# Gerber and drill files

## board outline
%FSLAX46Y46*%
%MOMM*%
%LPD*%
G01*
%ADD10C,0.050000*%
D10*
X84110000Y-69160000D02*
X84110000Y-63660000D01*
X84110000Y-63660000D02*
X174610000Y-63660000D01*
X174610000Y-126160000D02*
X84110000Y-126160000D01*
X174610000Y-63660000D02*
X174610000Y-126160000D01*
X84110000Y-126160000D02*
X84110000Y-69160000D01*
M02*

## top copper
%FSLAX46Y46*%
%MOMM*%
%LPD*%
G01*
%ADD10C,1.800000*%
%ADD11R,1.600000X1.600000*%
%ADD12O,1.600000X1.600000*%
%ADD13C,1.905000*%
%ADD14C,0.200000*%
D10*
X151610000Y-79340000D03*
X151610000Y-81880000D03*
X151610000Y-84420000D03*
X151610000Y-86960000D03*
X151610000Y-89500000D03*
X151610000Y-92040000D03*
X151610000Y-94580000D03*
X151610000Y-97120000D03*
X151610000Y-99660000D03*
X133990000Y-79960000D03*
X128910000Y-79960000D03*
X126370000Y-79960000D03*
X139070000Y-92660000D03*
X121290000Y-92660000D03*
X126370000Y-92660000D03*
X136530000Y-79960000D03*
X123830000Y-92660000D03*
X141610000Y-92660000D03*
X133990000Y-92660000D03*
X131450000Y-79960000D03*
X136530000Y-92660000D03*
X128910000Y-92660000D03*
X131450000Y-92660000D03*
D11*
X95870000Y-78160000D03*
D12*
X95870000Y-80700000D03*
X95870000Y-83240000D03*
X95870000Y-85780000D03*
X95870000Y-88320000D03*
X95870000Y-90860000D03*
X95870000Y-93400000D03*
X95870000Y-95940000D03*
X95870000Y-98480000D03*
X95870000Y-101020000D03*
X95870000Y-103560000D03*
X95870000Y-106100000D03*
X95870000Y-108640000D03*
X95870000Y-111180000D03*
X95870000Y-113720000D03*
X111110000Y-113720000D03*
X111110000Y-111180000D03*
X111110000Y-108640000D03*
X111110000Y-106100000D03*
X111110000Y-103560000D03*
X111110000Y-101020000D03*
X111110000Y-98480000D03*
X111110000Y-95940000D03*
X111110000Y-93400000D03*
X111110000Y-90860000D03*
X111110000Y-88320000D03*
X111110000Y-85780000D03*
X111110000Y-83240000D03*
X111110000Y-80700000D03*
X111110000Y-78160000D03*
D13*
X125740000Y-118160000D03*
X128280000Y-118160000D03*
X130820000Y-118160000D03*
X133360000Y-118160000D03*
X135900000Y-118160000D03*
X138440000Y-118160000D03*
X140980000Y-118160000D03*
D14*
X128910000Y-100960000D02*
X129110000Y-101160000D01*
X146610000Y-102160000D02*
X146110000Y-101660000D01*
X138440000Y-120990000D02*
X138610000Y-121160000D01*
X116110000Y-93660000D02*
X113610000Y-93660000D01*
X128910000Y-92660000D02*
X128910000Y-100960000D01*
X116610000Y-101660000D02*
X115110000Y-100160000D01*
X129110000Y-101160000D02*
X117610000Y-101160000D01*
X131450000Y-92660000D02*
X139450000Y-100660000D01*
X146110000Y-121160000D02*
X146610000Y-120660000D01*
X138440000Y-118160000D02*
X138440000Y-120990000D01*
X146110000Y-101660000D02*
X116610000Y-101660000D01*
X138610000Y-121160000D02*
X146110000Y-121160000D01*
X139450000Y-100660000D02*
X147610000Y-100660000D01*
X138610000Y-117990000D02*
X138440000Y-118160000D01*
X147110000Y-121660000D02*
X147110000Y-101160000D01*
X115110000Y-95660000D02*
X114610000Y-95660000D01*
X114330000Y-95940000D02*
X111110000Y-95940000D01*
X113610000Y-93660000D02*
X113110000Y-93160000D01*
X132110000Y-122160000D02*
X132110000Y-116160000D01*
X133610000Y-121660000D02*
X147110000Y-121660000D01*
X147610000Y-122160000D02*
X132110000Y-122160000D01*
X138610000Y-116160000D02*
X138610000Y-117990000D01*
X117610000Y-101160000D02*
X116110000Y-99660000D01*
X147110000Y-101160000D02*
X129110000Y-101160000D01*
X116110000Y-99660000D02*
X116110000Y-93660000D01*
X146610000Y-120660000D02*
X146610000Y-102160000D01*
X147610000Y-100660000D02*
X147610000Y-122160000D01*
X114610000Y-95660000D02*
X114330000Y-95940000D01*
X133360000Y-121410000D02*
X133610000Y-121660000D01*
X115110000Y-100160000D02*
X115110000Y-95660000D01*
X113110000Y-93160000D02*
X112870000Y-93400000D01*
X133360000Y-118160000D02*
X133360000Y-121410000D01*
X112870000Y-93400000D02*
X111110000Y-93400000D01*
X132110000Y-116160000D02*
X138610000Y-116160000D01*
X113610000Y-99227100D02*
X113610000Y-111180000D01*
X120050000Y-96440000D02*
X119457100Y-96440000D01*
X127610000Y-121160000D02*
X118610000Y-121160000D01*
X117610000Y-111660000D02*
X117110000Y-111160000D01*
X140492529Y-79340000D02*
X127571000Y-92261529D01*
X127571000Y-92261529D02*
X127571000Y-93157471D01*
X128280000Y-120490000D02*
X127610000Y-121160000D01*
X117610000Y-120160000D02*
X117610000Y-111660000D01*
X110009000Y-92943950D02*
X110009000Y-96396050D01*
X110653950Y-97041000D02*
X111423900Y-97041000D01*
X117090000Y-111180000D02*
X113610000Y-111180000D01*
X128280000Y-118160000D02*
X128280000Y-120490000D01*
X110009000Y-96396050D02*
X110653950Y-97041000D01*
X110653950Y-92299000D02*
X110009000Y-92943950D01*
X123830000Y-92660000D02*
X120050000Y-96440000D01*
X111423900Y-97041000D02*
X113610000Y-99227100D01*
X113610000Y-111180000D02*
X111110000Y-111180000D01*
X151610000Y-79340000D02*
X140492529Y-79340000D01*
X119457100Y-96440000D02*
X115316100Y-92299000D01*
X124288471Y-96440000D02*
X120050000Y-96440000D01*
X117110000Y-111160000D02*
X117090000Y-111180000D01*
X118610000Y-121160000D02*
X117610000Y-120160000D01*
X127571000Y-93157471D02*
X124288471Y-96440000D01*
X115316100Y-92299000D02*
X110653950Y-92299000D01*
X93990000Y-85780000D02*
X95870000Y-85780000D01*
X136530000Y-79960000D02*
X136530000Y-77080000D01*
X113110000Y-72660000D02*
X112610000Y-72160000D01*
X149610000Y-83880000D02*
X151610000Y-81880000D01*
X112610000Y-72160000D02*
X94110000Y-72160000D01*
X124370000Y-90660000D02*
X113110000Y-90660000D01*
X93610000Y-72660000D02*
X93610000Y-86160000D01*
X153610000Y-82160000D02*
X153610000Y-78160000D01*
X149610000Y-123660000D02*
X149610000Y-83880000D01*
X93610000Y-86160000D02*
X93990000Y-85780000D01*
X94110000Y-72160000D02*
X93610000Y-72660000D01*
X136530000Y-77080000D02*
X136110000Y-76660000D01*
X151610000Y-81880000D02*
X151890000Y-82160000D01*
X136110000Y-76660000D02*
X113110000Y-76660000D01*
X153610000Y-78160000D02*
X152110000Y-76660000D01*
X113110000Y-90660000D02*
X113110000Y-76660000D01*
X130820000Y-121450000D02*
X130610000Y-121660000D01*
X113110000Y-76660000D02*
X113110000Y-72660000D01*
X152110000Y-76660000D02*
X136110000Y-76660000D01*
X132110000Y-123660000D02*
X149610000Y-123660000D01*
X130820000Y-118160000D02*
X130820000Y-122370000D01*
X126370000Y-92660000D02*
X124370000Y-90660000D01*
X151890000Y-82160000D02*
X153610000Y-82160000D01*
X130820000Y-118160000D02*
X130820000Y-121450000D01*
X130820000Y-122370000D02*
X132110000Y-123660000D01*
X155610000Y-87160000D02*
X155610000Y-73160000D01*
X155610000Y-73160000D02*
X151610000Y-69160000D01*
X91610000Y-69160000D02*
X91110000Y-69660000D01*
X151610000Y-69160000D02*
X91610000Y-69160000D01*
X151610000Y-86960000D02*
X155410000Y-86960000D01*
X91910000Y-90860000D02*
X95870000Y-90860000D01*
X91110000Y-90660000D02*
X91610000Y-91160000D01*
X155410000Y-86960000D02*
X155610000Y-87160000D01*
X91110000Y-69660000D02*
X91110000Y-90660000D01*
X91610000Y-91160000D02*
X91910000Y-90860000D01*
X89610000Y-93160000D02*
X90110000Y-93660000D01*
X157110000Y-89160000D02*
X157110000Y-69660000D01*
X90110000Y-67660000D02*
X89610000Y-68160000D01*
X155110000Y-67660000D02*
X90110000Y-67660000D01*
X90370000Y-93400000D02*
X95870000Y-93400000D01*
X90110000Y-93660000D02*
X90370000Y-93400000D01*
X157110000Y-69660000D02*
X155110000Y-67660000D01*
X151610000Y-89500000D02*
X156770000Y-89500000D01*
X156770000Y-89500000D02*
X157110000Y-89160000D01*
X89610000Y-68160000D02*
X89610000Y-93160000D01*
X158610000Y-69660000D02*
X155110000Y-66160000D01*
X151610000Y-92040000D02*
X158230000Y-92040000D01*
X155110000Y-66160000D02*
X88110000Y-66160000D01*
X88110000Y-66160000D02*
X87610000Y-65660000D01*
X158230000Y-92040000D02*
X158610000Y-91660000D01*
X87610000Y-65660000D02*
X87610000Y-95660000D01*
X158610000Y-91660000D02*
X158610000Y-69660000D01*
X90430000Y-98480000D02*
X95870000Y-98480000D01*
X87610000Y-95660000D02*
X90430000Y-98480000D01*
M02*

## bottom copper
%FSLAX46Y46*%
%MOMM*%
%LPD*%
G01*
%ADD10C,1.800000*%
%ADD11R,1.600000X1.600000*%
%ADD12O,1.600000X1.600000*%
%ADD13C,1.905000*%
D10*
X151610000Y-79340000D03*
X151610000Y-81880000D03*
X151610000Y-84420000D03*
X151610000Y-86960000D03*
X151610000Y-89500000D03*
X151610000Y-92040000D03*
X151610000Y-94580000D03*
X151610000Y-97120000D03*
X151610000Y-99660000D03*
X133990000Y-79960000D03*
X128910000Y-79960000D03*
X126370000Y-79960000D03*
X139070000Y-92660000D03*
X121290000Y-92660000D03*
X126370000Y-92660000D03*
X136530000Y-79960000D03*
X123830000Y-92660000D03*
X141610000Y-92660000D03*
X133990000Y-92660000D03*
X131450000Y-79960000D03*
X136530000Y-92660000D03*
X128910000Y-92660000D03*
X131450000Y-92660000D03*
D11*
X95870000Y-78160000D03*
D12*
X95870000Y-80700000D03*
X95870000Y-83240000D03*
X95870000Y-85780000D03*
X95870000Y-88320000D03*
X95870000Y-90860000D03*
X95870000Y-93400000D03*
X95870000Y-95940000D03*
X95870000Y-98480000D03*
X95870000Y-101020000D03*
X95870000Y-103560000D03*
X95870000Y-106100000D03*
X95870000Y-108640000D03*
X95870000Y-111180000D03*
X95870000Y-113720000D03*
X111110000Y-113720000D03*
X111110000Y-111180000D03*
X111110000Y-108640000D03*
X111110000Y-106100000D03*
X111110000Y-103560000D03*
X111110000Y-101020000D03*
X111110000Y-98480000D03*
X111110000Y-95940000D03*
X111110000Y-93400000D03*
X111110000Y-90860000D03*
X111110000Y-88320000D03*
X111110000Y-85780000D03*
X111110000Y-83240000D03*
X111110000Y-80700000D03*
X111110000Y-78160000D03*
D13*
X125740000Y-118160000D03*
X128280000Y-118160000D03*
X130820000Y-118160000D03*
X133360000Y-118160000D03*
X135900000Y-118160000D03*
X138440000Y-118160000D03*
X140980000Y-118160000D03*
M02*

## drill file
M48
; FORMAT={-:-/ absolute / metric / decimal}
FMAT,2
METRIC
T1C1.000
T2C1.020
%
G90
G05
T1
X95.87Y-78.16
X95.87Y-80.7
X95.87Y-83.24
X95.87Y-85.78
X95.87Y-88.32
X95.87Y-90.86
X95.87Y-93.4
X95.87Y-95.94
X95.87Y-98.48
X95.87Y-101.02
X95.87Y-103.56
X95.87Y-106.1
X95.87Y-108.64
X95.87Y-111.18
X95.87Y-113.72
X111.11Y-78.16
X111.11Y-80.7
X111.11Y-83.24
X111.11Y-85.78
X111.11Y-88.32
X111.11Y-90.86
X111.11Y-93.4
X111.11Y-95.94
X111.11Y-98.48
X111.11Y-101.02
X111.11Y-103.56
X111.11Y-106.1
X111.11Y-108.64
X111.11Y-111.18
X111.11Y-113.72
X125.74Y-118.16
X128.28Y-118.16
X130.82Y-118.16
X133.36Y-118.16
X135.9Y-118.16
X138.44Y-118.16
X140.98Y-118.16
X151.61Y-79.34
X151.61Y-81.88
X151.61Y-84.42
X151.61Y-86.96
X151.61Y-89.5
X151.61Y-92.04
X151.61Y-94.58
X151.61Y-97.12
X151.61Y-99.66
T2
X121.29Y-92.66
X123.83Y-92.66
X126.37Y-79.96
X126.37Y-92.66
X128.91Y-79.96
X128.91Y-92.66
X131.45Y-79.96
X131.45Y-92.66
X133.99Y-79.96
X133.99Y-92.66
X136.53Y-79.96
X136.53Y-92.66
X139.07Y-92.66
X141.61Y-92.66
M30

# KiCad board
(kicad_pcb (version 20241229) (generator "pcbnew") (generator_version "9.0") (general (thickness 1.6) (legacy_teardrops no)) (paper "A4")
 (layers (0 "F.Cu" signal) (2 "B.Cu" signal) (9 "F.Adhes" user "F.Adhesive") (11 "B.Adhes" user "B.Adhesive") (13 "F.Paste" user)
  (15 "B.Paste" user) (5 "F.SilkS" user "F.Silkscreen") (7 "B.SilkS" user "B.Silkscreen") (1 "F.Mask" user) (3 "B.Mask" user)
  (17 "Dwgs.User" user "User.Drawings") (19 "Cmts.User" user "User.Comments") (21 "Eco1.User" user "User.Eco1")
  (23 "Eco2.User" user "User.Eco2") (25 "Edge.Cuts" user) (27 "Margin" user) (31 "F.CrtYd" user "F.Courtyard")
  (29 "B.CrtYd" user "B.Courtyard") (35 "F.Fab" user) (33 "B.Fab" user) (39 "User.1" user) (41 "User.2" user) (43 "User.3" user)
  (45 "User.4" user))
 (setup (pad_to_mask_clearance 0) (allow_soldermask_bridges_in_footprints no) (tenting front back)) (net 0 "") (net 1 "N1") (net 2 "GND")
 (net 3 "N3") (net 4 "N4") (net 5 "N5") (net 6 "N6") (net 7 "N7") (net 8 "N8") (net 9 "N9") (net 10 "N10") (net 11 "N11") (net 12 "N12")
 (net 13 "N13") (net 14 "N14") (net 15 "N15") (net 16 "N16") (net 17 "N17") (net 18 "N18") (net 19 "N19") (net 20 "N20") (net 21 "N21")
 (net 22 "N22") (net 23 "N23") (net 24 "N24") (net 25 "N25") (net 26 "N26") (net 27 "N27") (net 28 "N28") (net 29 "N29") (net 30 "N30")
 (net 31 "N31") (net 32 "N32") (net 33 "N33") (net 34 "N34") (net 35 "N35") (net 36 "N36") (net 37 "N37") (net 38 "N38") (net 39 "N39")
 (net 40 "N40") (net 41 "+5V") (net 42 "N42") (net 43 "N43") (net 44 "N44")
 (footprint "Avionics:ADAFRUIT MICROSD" (layer "F.Cu") (at 160.5 89.5 -90)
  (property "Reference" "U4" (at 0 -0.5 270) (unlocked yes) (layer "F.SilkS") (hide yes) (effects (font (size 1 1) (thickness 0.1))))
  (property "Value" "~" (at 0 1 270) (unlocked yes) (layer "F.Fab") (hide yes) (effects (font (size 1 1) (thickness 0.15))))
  (pad "1" thru_hole circle (at -10.16 8.89 270) (size 1.8 1.8) (drill 1) (layers "*.Cu" "*.Mask") (remove_unused_layers no) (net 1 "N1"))
  (pad "2" thru_hole circle (at -7.62 8.89 270) (size 1.8 1.8) (drill 1) (layers "*.Cu" "*.Mask") (remove_unused_layers no) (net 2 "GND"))
  (pad "3" thru_hole circle (at -5.08 8.89 270) (size 1.8 1.8) (drill 1) (layers "*.Cu" "*.Mask") (remove_unused_layers no) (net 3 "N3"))
  (pad "4" thru_hole circle (at -2.54 8.89 270) (size 1.8 1.8) (drill 1) (layers "*.Cu" "*.Mask") (remove_unused_layers no) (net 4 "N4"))
  (pad "5" thru_hole circle (at 0 8.89 270) (size 1.8 1.8) (drill 1) (layers "*.Cu" "*.Mask") (remove_unused_layers no) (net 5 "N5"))
  (pad "6" thru_hole circle (at 2.54 8.89 270) (size 1.8 1.8) (drill 1) (layers "*.Cu" "*.Mask") (remove_unused_layers no) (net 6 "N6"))
  (pad "7" thru_hole circle (at 5.08 8.89 270) (size 1.8 1.8) (drill 1) (layers "*.Cu" "*.Mask") (remove_unused_layers no) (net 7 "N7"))
  (pad "8" thru_hole circle (at 7.62 8.89 270) (size 1.8 1.8) (drill 1) (layers "*.Cu" "*.Mask") (remove_unused_layers no) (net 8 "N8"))
  (pad "9" thru_hole circle (at 10.16 8.89 270) (size 1.8 1.8) (drill 1) (layers "*.Cu" "*.Mask") (remove_unused_layers no) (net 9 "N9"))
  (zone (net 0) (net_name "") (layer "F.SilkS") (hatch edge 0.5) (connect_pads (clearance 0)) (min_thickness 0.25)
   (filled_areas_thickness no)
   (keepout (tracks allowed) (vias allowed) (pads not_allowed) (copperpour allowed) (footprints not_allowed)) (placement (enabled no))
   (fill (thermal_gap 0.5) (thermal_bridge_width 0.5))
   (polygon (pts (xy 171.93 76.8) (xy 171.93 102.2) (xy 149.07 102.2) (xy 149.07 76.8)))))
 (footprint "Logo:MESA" (layer "F.Cu") (at 161.61 114.16)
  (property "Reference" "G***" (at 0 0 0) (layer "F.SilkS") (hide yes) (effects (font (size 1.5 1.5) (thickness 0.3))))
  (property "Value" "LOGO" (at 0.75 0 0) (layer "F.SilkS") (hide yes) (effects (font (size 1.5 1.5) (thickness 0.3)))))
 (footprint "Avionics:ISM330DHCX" (layer "F.Cu") (at 131.45 86.31)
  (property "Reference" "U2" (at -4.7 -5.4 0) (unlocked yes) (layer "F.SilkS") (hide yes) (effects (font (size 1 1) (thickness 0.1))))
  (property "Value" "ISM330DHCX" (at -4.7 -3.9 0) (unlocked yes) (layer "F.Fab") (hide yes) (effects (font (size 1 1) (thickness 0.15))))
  (pad "1" thru_hole circle (at 2.54 -6.35) (size 1.8 1.8) (drill 1.02) (layers "*.Cu" "*.Mask") (remove_unused_layers no) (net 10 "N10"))
  (pad "2" thru_hole circle (at -2.54 -6.35) (size 1.8 1.8) (drill 1.02) (layers "*.Cu" "*.Mask") (remove_unused_layers no) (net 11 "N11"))
  (pad "3" thru_hole circle (at -5.08 -6.35) (size 1.8 1.8) (drill 1.02) (layers "*.Cu" "*.Mask") (remove_unused_layers no) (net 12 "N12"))
  (pad "4" thru_hole circle (at 7.62 6.35) (size 1.8 1.8) (drill 1.02) (layers "*.Cu" "*.Mask") (remove_unused_layers no) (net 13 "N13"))
  (pad "5" thru_hole circle (at -10.16 6.35) (size 1.8 1.8) (drill 1.02) (layers "*.Cu" "*.Mask") (remove_unused_layers no) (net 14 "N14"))
  (pad "6" thru_hole circle (at -5.08 6.35) (size 1.8 1.8) (drill 1.02) (layers "*.Cu" "*.Mask") (remove_unused_layers no) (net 2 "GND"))
  (pad "6" thru_hole circle (at 5.08 -6.35) (size 1.8 1.8) (drill 1.02) (layers "*.Cu" "*.Mask") (remove_unused_layers no) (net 2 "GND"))
  (pad "8" thru_hole circle (at -7.62 6.35) (size 1.8 1.8) (drill 1.02) (layers "*.Cu" "*.Mask") (remove_unused_layers no) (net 1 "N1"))
  (pad "9" thru_hole circle (at 10.16 6.35) (size 1.8 1.8) (drill 1.02) (layers "*.Cu" "*.Mask") (remove_unused_layers no) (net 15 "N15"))
  (pad "11" thru_hole circle (at 2.54 6.35) (size 1.8 1.8) (drill 1.02) (layers "*.Cu" "*.Mask") (remove_unused_layers no) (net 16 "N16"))
  (pad "12" thru_hole circle (at 0 -6.35) (size 1.8 1.8) (drill 1.02) (layers "*.Cu" "*.Mask") (remove_unused_layers no) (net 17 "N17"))
  (pad "12" thru_hole circle (at 5.08 6.35) (size 1.8 1.8) (drill 1.02) (layers "*.Cu" "*.Mask") (remove_unused_layers no) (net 17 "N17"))
  (pad "13" thru_hole circle (at -2.54 6.35) (size 1.8 1.8) (drill 1.02) (layers "*.Cu" "*.Mask") (remove_unused_layers no) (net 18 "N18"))
  (pad "14" thru_hole circle (at 0 6.35) (size 1.8 1.8) (drill 1.02) (layers "*.Cu" "*.Mask") (remove_unused_layers no) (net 18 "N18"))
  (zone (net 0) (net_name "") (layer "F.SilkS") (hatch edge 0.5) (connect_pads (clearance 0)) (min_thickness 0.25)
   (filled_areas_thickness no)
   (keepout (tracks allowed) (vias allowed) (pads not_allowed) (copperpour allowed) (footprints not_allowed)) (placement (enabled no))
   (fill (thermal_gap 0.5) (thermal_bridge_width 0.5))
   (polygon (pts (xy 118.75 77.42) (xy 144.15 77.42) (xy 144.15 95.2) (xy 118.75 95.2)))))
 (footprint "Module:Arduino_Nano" (layer "F.Cu") (at 95.87 78.16)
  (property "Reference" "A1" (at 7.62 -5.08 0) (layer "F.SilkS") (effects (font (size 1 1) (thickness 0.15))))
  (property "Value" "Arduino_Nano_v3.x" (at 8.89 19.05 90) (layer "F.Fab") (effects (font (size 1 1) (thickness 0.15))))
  (pad "1" thru_hole rect (at 0 0) (size 1.6 1.6) (drill 1) (layers "*.Cu" "*.Mask") (remove_unused_layers no) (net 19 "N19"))
  (pad "2" thru_hole oval (at 0 2.54) (size 1.6 1.6) (drill 1) (layers "*.Cu" "*.Mask") (remove_unused_layers no) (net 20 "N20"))
  (pad "3" thru_hole oval (at 0 5.08) (size 1.6 1.6) (drill 1) (layers "*.Cu" "*.Mask") (remove_unused_layers no) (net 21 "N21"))
  (pad "4" thru_hole oval (at 0 7.62) (size 1.6 1.6) (drill 1) (layers "*.Cu" "*.Mask") (remove_unused_layers no) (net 2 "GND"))
  (pad "5" thru_hole oval (at 0 10.16) (size 1.6 1.6) (drill 1) (layers "*.Cu" "*.Mask") (remove_unused_layers no) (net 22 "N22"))
  (pad "6" thru_hole oval (at 0 12.7) (size 1.6 1.6) (drill 1) (layers "*.Cu" "*.Mask") (remove_unused_layers no) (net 4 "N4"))
  (pad "7" thru_hole oval (at 0 15.24) (size 1.6 1.6) (drill 1) (layers "*.Cu" "*.Mask") (remove_unused_layers no) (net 5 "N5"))
  (pad "8" thru_hole oval (at 0 17.78) (size 1.6 1.6) (drill 1) (layers "*.Cu" "*.Mask") (remove_unused_layers no) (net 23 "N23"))
  (pad "9" thru_hole oval (at 0 20.32) (size 1.6 1.6) (drill 1) (layers "*.Cu" "*.Mask") (remove_unused_layers no) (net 6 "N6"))
  (pad "10" thru_hole oval (at 0 22.86) (size 1.6 1.6) (drill 1) (layers "*.Cu" "*.Mask") (remove_unused_layers no) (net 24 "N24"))
  (pad "11" thru_hole oval (at 0 25.4) (size 1.6 1.6) (drill 1) (layers "*.Cu" "*.Mask") (remove_unused_layers no) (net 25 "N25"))
  (pad "12" thru_hole oval (at 0 27.94) (size 1.6 1.6) (drill 1) (layers "*.Cu" "*.Mask") (remove_unused_layers no) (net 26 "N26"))
  (pad "13" thru_hole oval (at 0 30.48) (size 1.6 1.6) (drill 1) (layers "*.Cu" "*.Mask") (remove_unused_layers no) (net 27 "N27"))
  (pad "14" thru_hole oval (at 0 33.02) (size 1.6 1.6) (drill 1) (layers "*.Cu" "*.Mask") (remove_unused_layers no) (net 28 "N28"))
  (pad "15" thru_hole oval (at 0 35.56) (size 1.6 1.6) (drill 1) (layers "*.Cu" "*.Mask") (remove_unused_layers no) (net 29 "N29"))
  (pad "16" thru_hole oval (at 15.24 35.56) (size 1.6 1.6) (drill 1) (layers "*.Cu" "*.Mask") (remove_unused_layers no) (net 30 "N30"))
  (pad "17" thru_hole oval (at 15.24 33.02) (size 1.6 1.6) (drill 1) (layers "*.Cu" "*.Mask") (remove_unused_layers no) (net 1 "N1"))
  (pad "18" thru_hole oval (at 15.24 30.48) (size 1.6 1.6) (drill 1) (layers "*.Cu" "*.Mask") (remove_unused_layers no) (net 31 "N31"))
  (pad "19" thru_hole oval (at 15.24 27.94) (size 1.6 1.6) (drill 1) (layers "*.Cu" "*.Mask") (remove_unused_layers no) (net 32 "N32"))
  (pad "20" thru_hole oval (at 15.24 25.4) (size 1.6 1.6) (drill 1) (layers "*.Cu" "*.Mask") (remove_unused_layers no) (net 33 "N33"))
  (pad "21" thru_hole oval (at 15.24 22.86) (size 1.6 1.6) (drill 1) (layers "*.Cu" "*.Mask") (remove_unused_layers no) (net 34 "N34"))
  (pad "22" thru_hole oval (at 15.24 20.32) (size 1.6 1.6) (drill 1) (layers "*.Cu" "*.Mask") (remove_unused_layers no) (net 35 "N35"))
  (pad "23" thru_hole oval (at 15.24 17.78) (size 1.6 1.6) (drill 1) (layers "*.Cu" "*.Mask") (remove_unused_layers no) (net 18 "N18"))
  (pad "24" thru_hole oval (at 15.24 15.24) (size 1.6 1.6) (drill 1) (layers "*.Cu" "*.Mask") (remove_unused_layers no) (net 18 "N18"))
  (pad "25" thru_hole oval (at 15.24 12.7) (size 1.6 1.6) (drill 1) (layers "*.Cu" "*.Mask") (remove_unused_layers no) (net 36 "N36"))
  (pad "26" thru_hole oval (at 15.24 10.16) (size 1.6 1.6) (drill 1) (layers "*.Cu" "*.Mask") (remove_unused_layers no) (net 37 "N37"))
  (pad "27" thru_hole oval (at 15.24 7.62) (size 1.6 1.6) (drill 1) (layers "*.Cu" "*.Mask") (remove_unused_layers no) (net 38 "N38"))
  (pad "28" thru_hole oval (at 15.24 5.08) (size 1.6 1.6) (drill 1) (layers "*.Cu" "*.Mask") (remove_unused_layers no) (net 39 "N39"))
  (pad "29" thru_hole oval (at 15.24 2.54) (size 1.6 1.6) (drill 1) (layers "*.Cu" "*.Mask") (remove_unused_layers no) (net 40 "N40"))
  (pad "30" thru_hole oval (at 15.24 0) (size 1.6 1.6) (drill 1) (layers "*.Cu" "*.Mask") (remove_unused_layers no) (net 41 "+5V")))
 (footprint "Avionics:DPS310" (layer "F.Cu") (at 133.11 111.81)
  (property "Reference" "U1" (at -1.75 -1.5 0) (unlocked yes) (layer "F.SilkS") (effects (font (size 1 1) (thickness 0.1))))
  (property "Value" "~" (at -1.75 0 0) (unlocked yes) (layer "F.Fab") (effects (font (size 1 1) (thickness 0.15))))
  (pad "1" thru_hole circle (at -7.37 6.35) (size 1.905 1.905) (drill 1) (layers "*.Cu" "*.Mask") (remove_unused_layers no) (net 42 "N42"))
  (pad "2" thru_hole circle (at -4.83 6.35) (size 1.905 1.905) (drill 1) (layers "*.Cu" "*.Mask") (remove_unused_layers no) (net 1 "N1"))
  (pad "3" thru_hole circle (at -2.29 6.35) (size 1.905 1.905) (drill 1) (layers "*.Cu" "*.Mask") (remove_unused_layers no) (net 2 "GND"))
  (pad "4" thru_hole circle (at 0.25 6.35) (size 1.905 1.905) (drill 1) (layers "*.Cu" "*.Mask") (remove_unused_layers no) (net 18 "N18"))
  (pad "5" thru_hole circle (at 2.79 6.35) (size 1.905 1.905) (drill 1) (layers "*.Cu" "*.Mask") (remove_unused_layers no) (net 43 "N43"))
  (pad "6" thru_hole circle (at 5.33 6.35) (size 1.905 1.905) (drill 1) (layers "*.Cu" "*.Mask") (remove_unused_layers no) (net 18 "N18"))
  (pad "7" thru_hole circle (at 7.87 6.35) (size 1.905 1.905) (drill 1) (layers "*.Cu" "*.Mask") (remove_unused_layers no) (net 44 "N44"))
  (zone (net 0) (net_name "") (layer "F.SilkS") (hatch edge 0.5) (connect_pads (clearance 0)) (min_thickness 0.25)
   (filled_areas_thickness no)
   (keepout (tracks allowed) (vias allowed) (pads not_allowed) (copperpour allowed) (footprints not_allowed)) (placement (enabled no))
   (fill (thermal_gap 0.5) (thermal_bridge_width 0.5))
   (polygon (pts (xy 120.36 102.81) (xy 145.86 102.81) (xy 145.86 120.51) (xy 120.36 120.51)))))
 (gr_line (start 84.11 69.16) (end 84.11 63.66) (stroke (width 0.05) (type default)) (layer "Edge.Cuts"))
 (gr_line (start 84.11 63.66) (end 174.61 63.66) (stroke (width 0.05) (type default)) (layer "Edge.Cuts"))
 (gr_line (start 174.61 126.16) (end 84.11 126.16) (stroke (width 0.05) (type default)) (layer "Edge.Cuts"))
 (gr_line (start 174.61 63.66) (end 174.61 126.16) (stroke (width 0.05) (type default)) (layer "Edge.Cuts"))
 (gr_line (start 84.11 126.16) (end 84.11 69.16) (stroke (width 0.05) (type default)) (layer "Edge.Cuts"))
 (segment (start 128.91 100.96) (end 129.11 101.16) (width 0.2) (layer "F.Cu") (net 18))
 (segment (start 146.61 102.16) (end 146.11 101.66) (width 0.2) (layer "F.Cu") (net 18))
 (segment (start 138.44 120.99) (end 138.61 121.16) (width 0.2) (layer "F.Cu") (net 18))
 (segment (start 116.11 93.66) (end 113.61 93.66) (width 0.2) (layer "F.Cu") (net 18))
 (segment (start 128.91 92.66) (end 128.91 100.96) (width 0.2) (layer "F.Cu") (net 18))
 (segment (start 116.61 101.66) (end 115.11 100.16) (width 0.2) (layer "F.Cu") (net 18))
 (segment (start 129.11 101.16) (end 117.61 101.16) (width 0.2) (layer "F.Cu") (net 18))
 (segment (start 131.45 92.66) (end 139.45 100.66) (width 0.2) (layer "F.Cu") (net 18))
 (segment (start 146.11 121.16) (end 146.61 120.66) (width 0.2) (layer "F.Cu") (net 18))
 (segment (start 138.44 118.16) (end 138.44 120.99) (width 0.2) (layer "F.Cu") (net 18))
 (segment (start 146.11 101.66) (end 116.61 101.66) (width 0.2) (layer "F.Cu") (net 18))
 (segment (start 138.61 121.16) (end 146.11 121.16) (width 0.2) (layer "F.Cu") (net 18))
 (segment (start 139.45 100.66) (end 147.61 100.66) (width 0.2) (layer "F.Cu") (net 18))
 (segment (start 138.61 117.99) (end 138.44 118.16) (width 0.2) (layer "F.Cu") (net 18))
 (segment (start 147.11 121.66) (end 147.11 101.16) (width 0.2) (layer "F.Cu") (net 18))
 (segment (start 115.11 95.66) (end 114.61 95.66) (width 0.2) (layer "F.Cu") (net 18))
 (segment (start 114.33 95.94) (end 111.11 95.94) (width 0.2) (layer "F.Cu") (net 18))
 (segment (start 113.61 93.66) (end 113.11 93.16) (width 0.2) (layer "F.Cu") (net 18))
 (segment (start 132.11 122.16) (end 132.11 116.16) (width 0.2) (layer "F.Cu") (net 18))
 (segment (start 133.61 121.66) (end 147.11 121.66) (width 0.2) (layer "F.Cu") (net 18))
 (segment (start 147.61 122.16) (end 132.11 122.16) (width 0.2) (layer "F.Cu") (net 18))
 (segment (start 138.61 116.16) (end 138.61 117.99) (width 0.2) (layer "F.Cu") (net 18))
 (segment (start 117.61 101.16) (end 116.11 99.66) (width 0.2) (layer "F.Cu") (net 18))
 (segment (start 147.11 101.16) (end 129.11 101.16) (width 0.2) (layer "F.Cu") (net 18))
 (segment (start 116.11 99.66) (end 116.11 93.66) (width 0.2) (layer "F.Cu") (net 18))
 (segment (start 146.61 120.66) (end 146.61 102.16) (width 0.2) (layer "F.Cu") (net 18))
 (segment (start 147.61 100.66) (end 147.61 122.16) (width 0.2) (layer "F.Cu") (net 18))
 (segment (start 114.61 95.66) (end 114.33 95.94) (width 0.2) (layer "F.Cu") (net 18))
 (segment (start 133.36 121.41) (end 133.61 121.66) (width 0.2) (layer "F.Cu") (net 18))
 (segment (start 115.11 100.16) (end 115.11 95.66) (width 0.2) (layer "F.Cu") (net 18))
 (segment (start 113.11 93.16) (end 112.87 93.4) (width 0.2) (layer "F.Cu") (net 18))
 (segment (start 133.36 118.16) (end 133.36 121.41) (width 0.2) (layer "F.Cu") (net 18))
 (segment (start 112.87 93.4) (end 111.11 93.4) (width 0.2) (layer "F.Cu") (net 18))
 (segment (start 132.11 116.16) (end 138.61 116.16) (width 0.2) (layer "F.Cu") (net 18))
 (segment (start 113.61 99.2271) (end 113.61 111.18) (width 0.2) (layer "F.Cu") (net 1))
 (segment (start 120.05 96.44) (end 119.4571 96.44) (width 0.2) (layer "F.Cu") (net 1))
 (segment (start 127.61 121.16) (end 118.61 121.16) (width 0.2) (layer "F.Cu") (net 1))
 (segment (start 117.61 111.66) (end 117.11 111.16) (width 0.2) (layer "F.Cu") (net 1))
 (segment (start 140.492529 79.34) (end 127.571 92.261529) (width 0.2) (layer "F.Cu") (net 1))
 (segment (start 127.571 92.261529) (end 127.571 93.157471) (width 0.2) (layer "F.Cu") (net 1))
 (segment (start 128.28 120.49) (end 127.61 121.16) (width 0.2) (layer "F.Cu") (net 1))
 (segment (start 117.61 120.16) (end 117.61 111.66) (width 0.2) (layer "F.Cu") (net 1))
 (segment (start 110.009 92.94395) (end 110.009 96.39605) (width 0.2) (layer "F.Cu") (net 1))
 (segment (start 110.65395 97.041) (end 111.4239 97.041) (width 0.2) (layer "F.Cu") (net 1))
 (segment (start 117.09 111.18) (end 113.61 111.18) (width 0.2) (layer "F.Cu") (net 1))
 (segment (start 128.28 118.16) (end 128.28 120.49) (width 0.2) (layer "F.Cu") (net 1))
 (segment (start 110.009 96.39605) (end 110.65395 97.041) (width 0.2) (layer "F.Cu") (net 1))
 (segment (start 110.65395 92.299) (end 110.009 92.94395) (width 0.2) (layer "F.Cu") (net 1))
 (segment (start 123.83 92.66) (end 120.05 96.44) (width 0.2) (layer "F.Cu") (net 1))
 (segment (start 111.4239 97.041) (end 113.61 99.2271) (width 0.2) (layer "F.Cu") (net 1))
 (segment (start 113.61 111.18) (end 111.11 111.18) (width 0.2) (layer "F.Cu") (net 1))
 (segment (start 151.61 79.34) (end 140.492529 79.34) (width 0.2) (layer "F.Cu") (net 1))
 (segment (start 119.4571 96.44) (end 115.3161 92.299) (width 0.2) (layer "F.Cu") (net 1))
 (segment (start 124.288471 96.44) (end 120.05 96.44) (width 0.2) (layer "F.Cu") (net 1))
 (segment (start 117.11 111.16) (end 117.09 111.18) (width 0.2) (layer "F.Cu") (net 1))
 (segment (start 118.61 121.16) (end 117.61 120.16) (width 0.2) (layer "F.Cu") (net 1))
 (segment (start 127.571 93.157471) (end 124.288471 96.44) (width 0.2) (layer "F.Cu") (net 1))
 (segment (start 115.3161 92.299) (end 110.65395 92.299) (width 0.2) (layer "F.Cu") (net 1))
 (segment (start 93.99 85.78) (end 95.87 85.78) (width 0.2) (layer "F.Cu") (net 2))
 (segment (start 136.53 79.96) (end 136.53 77.08) (width 0.2) (layer "F.Cu") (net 2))
 (segment (start 113.11 72.66) (end 112.61 72.16) (width 0.2) (layer "F.Cu") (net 2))
 (segment (start 149.61 83.88) (end 151.61 81.88) (width 0.2) (layer "F.Cu") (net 2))
 (segment (start 112.61 72.16) (end 94.11 72.16) (width 0.2) (layer "F.Cu") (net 2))
 (segment (start 124.37 90.66) (end 113.11 90.66) (width 0.2) (layer "F.Cu") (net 2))
 (segment (start 93.61 72.66) (end 93.61 86.16) (width 0.2) (layer "F.Cu") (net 2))
 (segment (start 153.61 82.16) (end 153.61 78.16) (width 0.2) (layer "F.Cu") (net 2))
 (segment (start 149.61 123.66) (end 149.61 83.88) (width 0.2) (layer "F.Cu") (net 2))
 (segment (start 93.61 86.16) (end 93.99 85.78) (width 0.2) (layer "F.Cu") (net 2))
 (segment (start 94.11 72.16) (end 93.61 72.66) (width 0.2) (layer "F.Cu") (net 2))
 (segment (start 136.53 77.08) (end 136.11 76.66) (width 0.2) (layer "F.Cu") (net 2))
 (segment (start 151.61 81.88) (end 151.89 82.16) (width 0.2) (layer "F.Cu") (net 2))
 (segment (start 136.11 76.66) (end 113.11 76.66) (width 0.2) (layer "F.Cu") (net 2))
 (segment (start 153.61 78.16) (end 152.11 76.66) (width 0.2) (layer "F.Cu") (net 2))
 (segment (start 113.11 90.66) (end 113.11 76.66) (width 0.2) (layer "F.Cu") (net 2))
 (segment (start 130.82 121.45) (end 130.61 121.66) (width 0.2) (layer "F.Cu") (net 2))
 (segment (start 113.11 76.66) (end 113.11 72.66) (width 0.2) (layer "F.Cu") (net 2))
 (segment (start 152.11 76.66) (end 136.11 76.66) (width 0.2) (layer "F.Cu") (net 2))
 (segment (start 132.11 123.66) (end 149.61 123.66) (width 0.2) (layer "F.Cu") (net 2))
 (segment (start 130.82 118.16) (end 130.82 122.37) (width 0.2) (layer "F.Cu") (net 2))
 (segment (start 126.37 92.66) (end 124.37 90.66) (width 0.2) (layer "F.Cu") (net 2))
 (segment (start 151.89 82.16) (end 153.61 82.16) (width 0.2) (layer "F.Cu") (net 2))
 (segment (start 130.82 118.16) (end 130.82 121.45) (width 0.2) (layer "F.Cu") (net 2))
 (segment (start 130.82 122.37) (end 132.11 123.66) (width 0.2) (layer "F.Cu") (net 2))
 (segment (start 155.61 87.16) (end 155.61 73.16) (width 0.2) (layer "F.Cu") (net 4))
 (segment (start 155.61 73.16) (end 151.61 69.16) (width 0.2) (layer "F.Cu") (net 4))
 (segment (start 91.61 69.16) (end 91.11 69.66) (width 0.2) (layer "F.Cu") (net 4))
 (segment (start 151.61 69.16) (end 91.61 69.16) (width 0.2) (layer "F.Cu") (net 4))
 (segment (start 151.61 86.96) (end 155.41 86.96) (width 0.2) (layer "F.Cu") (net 4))
 (segment (start 91.91 90.86) (end 95.87 90.86) (width 0.2) (layer "F.Cu") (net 4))
 (segment (start 91.11 90.66) (end 91.61 91.16) (width 0.2) (layer "F.Cu") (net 4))
 (segment (start 155.41 86.96) (end 155.61 87.16) (width 0.2) (layer "F.Cu") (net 4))
 (segment (start 91.11 69.66) (end 91.11 90.66) (width 0.2) (layer "F.Cu") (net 4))
 (segment (start 91.61 91.16) (end 91.91 90.86) (width 0.2) (layer "F.Cu") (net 4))
 (segment (start 89.61 93.16) (end 90.11 93.66) (width 0.2) (layer "F.Cu") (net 5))
 (segment (start 157.11 89.16) (end 157.11 69.66) (width 0.2) (layer "F.Cu") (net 5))
 (segment (start 90.11 67.66) (end 89.61 68.16) (width 0.2) (layer "F.Cu") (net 5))
 (segment (start 155.11 67.66) (end 90.11 67.66) (width 0.2) (layer "F.Cu") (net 5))
 (segment (start 90.37 93.4) (end 95.87 93.4) (width 0.2) (layer "F.Cu") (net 5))
 (segment (start 90.11 93.66) (end 90.37 93.4) (width 0.2) (layer "F.Cu") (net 5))
 (segment (start 157.11 69.66) (end 155.11 67.66) (width 0.2) (layer "F.Cu") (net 5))
 (segment (start 151.61 89.5) (end 156.77 89.5) (width 0.2) (layer "F.Cu") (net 5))
 (segment (start 156.77 89.5) (end 157.11 89.16) (width 0.2) (layer "F.Cu") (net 5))
 (segment (start 89.61 68.16) (end 89.61 93.16) (width 0.2) (layer "F.Cu") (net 5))
 (segment (start 158.61 69.66) (end 155.11 66.16) (width 0.2) (layer "F.Cu") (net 6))
 (segment (start 151.61 92.04) (end 158.23 92.04) (width 0.2) (layer "F.Cu") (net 6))
 (segment (start 155.11 66.16) (end 88.11 66.16) (width 0.2) (layer "F.Cu") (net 6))
 (segment (start 88.11 66.16) (end 87.61 65.66) (width 0.2) (layer "F.Cu") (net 6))
 (segment (start 158.23 92.04) (end 158.61 91.66) (width 0.2) (layer "F.Cu") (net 6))
 (segment (start 87.61 65.66) (end 87.61 95.66) (width 0.2) (layer "F.Cu") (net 6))
 (segment (start 158.61 91.66) (end 158.61 69.66) (width 0.2) (layer "F.Cu") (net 6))
 (segment (start 90.43 98.48) (end 95.87 98.48) (width 0.2) (layer "F.Cu") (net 6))
 (segment (start 87.61 95.66) (end 90.43 98.48) (width 0.2) (layer "F.Cu") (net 6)))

